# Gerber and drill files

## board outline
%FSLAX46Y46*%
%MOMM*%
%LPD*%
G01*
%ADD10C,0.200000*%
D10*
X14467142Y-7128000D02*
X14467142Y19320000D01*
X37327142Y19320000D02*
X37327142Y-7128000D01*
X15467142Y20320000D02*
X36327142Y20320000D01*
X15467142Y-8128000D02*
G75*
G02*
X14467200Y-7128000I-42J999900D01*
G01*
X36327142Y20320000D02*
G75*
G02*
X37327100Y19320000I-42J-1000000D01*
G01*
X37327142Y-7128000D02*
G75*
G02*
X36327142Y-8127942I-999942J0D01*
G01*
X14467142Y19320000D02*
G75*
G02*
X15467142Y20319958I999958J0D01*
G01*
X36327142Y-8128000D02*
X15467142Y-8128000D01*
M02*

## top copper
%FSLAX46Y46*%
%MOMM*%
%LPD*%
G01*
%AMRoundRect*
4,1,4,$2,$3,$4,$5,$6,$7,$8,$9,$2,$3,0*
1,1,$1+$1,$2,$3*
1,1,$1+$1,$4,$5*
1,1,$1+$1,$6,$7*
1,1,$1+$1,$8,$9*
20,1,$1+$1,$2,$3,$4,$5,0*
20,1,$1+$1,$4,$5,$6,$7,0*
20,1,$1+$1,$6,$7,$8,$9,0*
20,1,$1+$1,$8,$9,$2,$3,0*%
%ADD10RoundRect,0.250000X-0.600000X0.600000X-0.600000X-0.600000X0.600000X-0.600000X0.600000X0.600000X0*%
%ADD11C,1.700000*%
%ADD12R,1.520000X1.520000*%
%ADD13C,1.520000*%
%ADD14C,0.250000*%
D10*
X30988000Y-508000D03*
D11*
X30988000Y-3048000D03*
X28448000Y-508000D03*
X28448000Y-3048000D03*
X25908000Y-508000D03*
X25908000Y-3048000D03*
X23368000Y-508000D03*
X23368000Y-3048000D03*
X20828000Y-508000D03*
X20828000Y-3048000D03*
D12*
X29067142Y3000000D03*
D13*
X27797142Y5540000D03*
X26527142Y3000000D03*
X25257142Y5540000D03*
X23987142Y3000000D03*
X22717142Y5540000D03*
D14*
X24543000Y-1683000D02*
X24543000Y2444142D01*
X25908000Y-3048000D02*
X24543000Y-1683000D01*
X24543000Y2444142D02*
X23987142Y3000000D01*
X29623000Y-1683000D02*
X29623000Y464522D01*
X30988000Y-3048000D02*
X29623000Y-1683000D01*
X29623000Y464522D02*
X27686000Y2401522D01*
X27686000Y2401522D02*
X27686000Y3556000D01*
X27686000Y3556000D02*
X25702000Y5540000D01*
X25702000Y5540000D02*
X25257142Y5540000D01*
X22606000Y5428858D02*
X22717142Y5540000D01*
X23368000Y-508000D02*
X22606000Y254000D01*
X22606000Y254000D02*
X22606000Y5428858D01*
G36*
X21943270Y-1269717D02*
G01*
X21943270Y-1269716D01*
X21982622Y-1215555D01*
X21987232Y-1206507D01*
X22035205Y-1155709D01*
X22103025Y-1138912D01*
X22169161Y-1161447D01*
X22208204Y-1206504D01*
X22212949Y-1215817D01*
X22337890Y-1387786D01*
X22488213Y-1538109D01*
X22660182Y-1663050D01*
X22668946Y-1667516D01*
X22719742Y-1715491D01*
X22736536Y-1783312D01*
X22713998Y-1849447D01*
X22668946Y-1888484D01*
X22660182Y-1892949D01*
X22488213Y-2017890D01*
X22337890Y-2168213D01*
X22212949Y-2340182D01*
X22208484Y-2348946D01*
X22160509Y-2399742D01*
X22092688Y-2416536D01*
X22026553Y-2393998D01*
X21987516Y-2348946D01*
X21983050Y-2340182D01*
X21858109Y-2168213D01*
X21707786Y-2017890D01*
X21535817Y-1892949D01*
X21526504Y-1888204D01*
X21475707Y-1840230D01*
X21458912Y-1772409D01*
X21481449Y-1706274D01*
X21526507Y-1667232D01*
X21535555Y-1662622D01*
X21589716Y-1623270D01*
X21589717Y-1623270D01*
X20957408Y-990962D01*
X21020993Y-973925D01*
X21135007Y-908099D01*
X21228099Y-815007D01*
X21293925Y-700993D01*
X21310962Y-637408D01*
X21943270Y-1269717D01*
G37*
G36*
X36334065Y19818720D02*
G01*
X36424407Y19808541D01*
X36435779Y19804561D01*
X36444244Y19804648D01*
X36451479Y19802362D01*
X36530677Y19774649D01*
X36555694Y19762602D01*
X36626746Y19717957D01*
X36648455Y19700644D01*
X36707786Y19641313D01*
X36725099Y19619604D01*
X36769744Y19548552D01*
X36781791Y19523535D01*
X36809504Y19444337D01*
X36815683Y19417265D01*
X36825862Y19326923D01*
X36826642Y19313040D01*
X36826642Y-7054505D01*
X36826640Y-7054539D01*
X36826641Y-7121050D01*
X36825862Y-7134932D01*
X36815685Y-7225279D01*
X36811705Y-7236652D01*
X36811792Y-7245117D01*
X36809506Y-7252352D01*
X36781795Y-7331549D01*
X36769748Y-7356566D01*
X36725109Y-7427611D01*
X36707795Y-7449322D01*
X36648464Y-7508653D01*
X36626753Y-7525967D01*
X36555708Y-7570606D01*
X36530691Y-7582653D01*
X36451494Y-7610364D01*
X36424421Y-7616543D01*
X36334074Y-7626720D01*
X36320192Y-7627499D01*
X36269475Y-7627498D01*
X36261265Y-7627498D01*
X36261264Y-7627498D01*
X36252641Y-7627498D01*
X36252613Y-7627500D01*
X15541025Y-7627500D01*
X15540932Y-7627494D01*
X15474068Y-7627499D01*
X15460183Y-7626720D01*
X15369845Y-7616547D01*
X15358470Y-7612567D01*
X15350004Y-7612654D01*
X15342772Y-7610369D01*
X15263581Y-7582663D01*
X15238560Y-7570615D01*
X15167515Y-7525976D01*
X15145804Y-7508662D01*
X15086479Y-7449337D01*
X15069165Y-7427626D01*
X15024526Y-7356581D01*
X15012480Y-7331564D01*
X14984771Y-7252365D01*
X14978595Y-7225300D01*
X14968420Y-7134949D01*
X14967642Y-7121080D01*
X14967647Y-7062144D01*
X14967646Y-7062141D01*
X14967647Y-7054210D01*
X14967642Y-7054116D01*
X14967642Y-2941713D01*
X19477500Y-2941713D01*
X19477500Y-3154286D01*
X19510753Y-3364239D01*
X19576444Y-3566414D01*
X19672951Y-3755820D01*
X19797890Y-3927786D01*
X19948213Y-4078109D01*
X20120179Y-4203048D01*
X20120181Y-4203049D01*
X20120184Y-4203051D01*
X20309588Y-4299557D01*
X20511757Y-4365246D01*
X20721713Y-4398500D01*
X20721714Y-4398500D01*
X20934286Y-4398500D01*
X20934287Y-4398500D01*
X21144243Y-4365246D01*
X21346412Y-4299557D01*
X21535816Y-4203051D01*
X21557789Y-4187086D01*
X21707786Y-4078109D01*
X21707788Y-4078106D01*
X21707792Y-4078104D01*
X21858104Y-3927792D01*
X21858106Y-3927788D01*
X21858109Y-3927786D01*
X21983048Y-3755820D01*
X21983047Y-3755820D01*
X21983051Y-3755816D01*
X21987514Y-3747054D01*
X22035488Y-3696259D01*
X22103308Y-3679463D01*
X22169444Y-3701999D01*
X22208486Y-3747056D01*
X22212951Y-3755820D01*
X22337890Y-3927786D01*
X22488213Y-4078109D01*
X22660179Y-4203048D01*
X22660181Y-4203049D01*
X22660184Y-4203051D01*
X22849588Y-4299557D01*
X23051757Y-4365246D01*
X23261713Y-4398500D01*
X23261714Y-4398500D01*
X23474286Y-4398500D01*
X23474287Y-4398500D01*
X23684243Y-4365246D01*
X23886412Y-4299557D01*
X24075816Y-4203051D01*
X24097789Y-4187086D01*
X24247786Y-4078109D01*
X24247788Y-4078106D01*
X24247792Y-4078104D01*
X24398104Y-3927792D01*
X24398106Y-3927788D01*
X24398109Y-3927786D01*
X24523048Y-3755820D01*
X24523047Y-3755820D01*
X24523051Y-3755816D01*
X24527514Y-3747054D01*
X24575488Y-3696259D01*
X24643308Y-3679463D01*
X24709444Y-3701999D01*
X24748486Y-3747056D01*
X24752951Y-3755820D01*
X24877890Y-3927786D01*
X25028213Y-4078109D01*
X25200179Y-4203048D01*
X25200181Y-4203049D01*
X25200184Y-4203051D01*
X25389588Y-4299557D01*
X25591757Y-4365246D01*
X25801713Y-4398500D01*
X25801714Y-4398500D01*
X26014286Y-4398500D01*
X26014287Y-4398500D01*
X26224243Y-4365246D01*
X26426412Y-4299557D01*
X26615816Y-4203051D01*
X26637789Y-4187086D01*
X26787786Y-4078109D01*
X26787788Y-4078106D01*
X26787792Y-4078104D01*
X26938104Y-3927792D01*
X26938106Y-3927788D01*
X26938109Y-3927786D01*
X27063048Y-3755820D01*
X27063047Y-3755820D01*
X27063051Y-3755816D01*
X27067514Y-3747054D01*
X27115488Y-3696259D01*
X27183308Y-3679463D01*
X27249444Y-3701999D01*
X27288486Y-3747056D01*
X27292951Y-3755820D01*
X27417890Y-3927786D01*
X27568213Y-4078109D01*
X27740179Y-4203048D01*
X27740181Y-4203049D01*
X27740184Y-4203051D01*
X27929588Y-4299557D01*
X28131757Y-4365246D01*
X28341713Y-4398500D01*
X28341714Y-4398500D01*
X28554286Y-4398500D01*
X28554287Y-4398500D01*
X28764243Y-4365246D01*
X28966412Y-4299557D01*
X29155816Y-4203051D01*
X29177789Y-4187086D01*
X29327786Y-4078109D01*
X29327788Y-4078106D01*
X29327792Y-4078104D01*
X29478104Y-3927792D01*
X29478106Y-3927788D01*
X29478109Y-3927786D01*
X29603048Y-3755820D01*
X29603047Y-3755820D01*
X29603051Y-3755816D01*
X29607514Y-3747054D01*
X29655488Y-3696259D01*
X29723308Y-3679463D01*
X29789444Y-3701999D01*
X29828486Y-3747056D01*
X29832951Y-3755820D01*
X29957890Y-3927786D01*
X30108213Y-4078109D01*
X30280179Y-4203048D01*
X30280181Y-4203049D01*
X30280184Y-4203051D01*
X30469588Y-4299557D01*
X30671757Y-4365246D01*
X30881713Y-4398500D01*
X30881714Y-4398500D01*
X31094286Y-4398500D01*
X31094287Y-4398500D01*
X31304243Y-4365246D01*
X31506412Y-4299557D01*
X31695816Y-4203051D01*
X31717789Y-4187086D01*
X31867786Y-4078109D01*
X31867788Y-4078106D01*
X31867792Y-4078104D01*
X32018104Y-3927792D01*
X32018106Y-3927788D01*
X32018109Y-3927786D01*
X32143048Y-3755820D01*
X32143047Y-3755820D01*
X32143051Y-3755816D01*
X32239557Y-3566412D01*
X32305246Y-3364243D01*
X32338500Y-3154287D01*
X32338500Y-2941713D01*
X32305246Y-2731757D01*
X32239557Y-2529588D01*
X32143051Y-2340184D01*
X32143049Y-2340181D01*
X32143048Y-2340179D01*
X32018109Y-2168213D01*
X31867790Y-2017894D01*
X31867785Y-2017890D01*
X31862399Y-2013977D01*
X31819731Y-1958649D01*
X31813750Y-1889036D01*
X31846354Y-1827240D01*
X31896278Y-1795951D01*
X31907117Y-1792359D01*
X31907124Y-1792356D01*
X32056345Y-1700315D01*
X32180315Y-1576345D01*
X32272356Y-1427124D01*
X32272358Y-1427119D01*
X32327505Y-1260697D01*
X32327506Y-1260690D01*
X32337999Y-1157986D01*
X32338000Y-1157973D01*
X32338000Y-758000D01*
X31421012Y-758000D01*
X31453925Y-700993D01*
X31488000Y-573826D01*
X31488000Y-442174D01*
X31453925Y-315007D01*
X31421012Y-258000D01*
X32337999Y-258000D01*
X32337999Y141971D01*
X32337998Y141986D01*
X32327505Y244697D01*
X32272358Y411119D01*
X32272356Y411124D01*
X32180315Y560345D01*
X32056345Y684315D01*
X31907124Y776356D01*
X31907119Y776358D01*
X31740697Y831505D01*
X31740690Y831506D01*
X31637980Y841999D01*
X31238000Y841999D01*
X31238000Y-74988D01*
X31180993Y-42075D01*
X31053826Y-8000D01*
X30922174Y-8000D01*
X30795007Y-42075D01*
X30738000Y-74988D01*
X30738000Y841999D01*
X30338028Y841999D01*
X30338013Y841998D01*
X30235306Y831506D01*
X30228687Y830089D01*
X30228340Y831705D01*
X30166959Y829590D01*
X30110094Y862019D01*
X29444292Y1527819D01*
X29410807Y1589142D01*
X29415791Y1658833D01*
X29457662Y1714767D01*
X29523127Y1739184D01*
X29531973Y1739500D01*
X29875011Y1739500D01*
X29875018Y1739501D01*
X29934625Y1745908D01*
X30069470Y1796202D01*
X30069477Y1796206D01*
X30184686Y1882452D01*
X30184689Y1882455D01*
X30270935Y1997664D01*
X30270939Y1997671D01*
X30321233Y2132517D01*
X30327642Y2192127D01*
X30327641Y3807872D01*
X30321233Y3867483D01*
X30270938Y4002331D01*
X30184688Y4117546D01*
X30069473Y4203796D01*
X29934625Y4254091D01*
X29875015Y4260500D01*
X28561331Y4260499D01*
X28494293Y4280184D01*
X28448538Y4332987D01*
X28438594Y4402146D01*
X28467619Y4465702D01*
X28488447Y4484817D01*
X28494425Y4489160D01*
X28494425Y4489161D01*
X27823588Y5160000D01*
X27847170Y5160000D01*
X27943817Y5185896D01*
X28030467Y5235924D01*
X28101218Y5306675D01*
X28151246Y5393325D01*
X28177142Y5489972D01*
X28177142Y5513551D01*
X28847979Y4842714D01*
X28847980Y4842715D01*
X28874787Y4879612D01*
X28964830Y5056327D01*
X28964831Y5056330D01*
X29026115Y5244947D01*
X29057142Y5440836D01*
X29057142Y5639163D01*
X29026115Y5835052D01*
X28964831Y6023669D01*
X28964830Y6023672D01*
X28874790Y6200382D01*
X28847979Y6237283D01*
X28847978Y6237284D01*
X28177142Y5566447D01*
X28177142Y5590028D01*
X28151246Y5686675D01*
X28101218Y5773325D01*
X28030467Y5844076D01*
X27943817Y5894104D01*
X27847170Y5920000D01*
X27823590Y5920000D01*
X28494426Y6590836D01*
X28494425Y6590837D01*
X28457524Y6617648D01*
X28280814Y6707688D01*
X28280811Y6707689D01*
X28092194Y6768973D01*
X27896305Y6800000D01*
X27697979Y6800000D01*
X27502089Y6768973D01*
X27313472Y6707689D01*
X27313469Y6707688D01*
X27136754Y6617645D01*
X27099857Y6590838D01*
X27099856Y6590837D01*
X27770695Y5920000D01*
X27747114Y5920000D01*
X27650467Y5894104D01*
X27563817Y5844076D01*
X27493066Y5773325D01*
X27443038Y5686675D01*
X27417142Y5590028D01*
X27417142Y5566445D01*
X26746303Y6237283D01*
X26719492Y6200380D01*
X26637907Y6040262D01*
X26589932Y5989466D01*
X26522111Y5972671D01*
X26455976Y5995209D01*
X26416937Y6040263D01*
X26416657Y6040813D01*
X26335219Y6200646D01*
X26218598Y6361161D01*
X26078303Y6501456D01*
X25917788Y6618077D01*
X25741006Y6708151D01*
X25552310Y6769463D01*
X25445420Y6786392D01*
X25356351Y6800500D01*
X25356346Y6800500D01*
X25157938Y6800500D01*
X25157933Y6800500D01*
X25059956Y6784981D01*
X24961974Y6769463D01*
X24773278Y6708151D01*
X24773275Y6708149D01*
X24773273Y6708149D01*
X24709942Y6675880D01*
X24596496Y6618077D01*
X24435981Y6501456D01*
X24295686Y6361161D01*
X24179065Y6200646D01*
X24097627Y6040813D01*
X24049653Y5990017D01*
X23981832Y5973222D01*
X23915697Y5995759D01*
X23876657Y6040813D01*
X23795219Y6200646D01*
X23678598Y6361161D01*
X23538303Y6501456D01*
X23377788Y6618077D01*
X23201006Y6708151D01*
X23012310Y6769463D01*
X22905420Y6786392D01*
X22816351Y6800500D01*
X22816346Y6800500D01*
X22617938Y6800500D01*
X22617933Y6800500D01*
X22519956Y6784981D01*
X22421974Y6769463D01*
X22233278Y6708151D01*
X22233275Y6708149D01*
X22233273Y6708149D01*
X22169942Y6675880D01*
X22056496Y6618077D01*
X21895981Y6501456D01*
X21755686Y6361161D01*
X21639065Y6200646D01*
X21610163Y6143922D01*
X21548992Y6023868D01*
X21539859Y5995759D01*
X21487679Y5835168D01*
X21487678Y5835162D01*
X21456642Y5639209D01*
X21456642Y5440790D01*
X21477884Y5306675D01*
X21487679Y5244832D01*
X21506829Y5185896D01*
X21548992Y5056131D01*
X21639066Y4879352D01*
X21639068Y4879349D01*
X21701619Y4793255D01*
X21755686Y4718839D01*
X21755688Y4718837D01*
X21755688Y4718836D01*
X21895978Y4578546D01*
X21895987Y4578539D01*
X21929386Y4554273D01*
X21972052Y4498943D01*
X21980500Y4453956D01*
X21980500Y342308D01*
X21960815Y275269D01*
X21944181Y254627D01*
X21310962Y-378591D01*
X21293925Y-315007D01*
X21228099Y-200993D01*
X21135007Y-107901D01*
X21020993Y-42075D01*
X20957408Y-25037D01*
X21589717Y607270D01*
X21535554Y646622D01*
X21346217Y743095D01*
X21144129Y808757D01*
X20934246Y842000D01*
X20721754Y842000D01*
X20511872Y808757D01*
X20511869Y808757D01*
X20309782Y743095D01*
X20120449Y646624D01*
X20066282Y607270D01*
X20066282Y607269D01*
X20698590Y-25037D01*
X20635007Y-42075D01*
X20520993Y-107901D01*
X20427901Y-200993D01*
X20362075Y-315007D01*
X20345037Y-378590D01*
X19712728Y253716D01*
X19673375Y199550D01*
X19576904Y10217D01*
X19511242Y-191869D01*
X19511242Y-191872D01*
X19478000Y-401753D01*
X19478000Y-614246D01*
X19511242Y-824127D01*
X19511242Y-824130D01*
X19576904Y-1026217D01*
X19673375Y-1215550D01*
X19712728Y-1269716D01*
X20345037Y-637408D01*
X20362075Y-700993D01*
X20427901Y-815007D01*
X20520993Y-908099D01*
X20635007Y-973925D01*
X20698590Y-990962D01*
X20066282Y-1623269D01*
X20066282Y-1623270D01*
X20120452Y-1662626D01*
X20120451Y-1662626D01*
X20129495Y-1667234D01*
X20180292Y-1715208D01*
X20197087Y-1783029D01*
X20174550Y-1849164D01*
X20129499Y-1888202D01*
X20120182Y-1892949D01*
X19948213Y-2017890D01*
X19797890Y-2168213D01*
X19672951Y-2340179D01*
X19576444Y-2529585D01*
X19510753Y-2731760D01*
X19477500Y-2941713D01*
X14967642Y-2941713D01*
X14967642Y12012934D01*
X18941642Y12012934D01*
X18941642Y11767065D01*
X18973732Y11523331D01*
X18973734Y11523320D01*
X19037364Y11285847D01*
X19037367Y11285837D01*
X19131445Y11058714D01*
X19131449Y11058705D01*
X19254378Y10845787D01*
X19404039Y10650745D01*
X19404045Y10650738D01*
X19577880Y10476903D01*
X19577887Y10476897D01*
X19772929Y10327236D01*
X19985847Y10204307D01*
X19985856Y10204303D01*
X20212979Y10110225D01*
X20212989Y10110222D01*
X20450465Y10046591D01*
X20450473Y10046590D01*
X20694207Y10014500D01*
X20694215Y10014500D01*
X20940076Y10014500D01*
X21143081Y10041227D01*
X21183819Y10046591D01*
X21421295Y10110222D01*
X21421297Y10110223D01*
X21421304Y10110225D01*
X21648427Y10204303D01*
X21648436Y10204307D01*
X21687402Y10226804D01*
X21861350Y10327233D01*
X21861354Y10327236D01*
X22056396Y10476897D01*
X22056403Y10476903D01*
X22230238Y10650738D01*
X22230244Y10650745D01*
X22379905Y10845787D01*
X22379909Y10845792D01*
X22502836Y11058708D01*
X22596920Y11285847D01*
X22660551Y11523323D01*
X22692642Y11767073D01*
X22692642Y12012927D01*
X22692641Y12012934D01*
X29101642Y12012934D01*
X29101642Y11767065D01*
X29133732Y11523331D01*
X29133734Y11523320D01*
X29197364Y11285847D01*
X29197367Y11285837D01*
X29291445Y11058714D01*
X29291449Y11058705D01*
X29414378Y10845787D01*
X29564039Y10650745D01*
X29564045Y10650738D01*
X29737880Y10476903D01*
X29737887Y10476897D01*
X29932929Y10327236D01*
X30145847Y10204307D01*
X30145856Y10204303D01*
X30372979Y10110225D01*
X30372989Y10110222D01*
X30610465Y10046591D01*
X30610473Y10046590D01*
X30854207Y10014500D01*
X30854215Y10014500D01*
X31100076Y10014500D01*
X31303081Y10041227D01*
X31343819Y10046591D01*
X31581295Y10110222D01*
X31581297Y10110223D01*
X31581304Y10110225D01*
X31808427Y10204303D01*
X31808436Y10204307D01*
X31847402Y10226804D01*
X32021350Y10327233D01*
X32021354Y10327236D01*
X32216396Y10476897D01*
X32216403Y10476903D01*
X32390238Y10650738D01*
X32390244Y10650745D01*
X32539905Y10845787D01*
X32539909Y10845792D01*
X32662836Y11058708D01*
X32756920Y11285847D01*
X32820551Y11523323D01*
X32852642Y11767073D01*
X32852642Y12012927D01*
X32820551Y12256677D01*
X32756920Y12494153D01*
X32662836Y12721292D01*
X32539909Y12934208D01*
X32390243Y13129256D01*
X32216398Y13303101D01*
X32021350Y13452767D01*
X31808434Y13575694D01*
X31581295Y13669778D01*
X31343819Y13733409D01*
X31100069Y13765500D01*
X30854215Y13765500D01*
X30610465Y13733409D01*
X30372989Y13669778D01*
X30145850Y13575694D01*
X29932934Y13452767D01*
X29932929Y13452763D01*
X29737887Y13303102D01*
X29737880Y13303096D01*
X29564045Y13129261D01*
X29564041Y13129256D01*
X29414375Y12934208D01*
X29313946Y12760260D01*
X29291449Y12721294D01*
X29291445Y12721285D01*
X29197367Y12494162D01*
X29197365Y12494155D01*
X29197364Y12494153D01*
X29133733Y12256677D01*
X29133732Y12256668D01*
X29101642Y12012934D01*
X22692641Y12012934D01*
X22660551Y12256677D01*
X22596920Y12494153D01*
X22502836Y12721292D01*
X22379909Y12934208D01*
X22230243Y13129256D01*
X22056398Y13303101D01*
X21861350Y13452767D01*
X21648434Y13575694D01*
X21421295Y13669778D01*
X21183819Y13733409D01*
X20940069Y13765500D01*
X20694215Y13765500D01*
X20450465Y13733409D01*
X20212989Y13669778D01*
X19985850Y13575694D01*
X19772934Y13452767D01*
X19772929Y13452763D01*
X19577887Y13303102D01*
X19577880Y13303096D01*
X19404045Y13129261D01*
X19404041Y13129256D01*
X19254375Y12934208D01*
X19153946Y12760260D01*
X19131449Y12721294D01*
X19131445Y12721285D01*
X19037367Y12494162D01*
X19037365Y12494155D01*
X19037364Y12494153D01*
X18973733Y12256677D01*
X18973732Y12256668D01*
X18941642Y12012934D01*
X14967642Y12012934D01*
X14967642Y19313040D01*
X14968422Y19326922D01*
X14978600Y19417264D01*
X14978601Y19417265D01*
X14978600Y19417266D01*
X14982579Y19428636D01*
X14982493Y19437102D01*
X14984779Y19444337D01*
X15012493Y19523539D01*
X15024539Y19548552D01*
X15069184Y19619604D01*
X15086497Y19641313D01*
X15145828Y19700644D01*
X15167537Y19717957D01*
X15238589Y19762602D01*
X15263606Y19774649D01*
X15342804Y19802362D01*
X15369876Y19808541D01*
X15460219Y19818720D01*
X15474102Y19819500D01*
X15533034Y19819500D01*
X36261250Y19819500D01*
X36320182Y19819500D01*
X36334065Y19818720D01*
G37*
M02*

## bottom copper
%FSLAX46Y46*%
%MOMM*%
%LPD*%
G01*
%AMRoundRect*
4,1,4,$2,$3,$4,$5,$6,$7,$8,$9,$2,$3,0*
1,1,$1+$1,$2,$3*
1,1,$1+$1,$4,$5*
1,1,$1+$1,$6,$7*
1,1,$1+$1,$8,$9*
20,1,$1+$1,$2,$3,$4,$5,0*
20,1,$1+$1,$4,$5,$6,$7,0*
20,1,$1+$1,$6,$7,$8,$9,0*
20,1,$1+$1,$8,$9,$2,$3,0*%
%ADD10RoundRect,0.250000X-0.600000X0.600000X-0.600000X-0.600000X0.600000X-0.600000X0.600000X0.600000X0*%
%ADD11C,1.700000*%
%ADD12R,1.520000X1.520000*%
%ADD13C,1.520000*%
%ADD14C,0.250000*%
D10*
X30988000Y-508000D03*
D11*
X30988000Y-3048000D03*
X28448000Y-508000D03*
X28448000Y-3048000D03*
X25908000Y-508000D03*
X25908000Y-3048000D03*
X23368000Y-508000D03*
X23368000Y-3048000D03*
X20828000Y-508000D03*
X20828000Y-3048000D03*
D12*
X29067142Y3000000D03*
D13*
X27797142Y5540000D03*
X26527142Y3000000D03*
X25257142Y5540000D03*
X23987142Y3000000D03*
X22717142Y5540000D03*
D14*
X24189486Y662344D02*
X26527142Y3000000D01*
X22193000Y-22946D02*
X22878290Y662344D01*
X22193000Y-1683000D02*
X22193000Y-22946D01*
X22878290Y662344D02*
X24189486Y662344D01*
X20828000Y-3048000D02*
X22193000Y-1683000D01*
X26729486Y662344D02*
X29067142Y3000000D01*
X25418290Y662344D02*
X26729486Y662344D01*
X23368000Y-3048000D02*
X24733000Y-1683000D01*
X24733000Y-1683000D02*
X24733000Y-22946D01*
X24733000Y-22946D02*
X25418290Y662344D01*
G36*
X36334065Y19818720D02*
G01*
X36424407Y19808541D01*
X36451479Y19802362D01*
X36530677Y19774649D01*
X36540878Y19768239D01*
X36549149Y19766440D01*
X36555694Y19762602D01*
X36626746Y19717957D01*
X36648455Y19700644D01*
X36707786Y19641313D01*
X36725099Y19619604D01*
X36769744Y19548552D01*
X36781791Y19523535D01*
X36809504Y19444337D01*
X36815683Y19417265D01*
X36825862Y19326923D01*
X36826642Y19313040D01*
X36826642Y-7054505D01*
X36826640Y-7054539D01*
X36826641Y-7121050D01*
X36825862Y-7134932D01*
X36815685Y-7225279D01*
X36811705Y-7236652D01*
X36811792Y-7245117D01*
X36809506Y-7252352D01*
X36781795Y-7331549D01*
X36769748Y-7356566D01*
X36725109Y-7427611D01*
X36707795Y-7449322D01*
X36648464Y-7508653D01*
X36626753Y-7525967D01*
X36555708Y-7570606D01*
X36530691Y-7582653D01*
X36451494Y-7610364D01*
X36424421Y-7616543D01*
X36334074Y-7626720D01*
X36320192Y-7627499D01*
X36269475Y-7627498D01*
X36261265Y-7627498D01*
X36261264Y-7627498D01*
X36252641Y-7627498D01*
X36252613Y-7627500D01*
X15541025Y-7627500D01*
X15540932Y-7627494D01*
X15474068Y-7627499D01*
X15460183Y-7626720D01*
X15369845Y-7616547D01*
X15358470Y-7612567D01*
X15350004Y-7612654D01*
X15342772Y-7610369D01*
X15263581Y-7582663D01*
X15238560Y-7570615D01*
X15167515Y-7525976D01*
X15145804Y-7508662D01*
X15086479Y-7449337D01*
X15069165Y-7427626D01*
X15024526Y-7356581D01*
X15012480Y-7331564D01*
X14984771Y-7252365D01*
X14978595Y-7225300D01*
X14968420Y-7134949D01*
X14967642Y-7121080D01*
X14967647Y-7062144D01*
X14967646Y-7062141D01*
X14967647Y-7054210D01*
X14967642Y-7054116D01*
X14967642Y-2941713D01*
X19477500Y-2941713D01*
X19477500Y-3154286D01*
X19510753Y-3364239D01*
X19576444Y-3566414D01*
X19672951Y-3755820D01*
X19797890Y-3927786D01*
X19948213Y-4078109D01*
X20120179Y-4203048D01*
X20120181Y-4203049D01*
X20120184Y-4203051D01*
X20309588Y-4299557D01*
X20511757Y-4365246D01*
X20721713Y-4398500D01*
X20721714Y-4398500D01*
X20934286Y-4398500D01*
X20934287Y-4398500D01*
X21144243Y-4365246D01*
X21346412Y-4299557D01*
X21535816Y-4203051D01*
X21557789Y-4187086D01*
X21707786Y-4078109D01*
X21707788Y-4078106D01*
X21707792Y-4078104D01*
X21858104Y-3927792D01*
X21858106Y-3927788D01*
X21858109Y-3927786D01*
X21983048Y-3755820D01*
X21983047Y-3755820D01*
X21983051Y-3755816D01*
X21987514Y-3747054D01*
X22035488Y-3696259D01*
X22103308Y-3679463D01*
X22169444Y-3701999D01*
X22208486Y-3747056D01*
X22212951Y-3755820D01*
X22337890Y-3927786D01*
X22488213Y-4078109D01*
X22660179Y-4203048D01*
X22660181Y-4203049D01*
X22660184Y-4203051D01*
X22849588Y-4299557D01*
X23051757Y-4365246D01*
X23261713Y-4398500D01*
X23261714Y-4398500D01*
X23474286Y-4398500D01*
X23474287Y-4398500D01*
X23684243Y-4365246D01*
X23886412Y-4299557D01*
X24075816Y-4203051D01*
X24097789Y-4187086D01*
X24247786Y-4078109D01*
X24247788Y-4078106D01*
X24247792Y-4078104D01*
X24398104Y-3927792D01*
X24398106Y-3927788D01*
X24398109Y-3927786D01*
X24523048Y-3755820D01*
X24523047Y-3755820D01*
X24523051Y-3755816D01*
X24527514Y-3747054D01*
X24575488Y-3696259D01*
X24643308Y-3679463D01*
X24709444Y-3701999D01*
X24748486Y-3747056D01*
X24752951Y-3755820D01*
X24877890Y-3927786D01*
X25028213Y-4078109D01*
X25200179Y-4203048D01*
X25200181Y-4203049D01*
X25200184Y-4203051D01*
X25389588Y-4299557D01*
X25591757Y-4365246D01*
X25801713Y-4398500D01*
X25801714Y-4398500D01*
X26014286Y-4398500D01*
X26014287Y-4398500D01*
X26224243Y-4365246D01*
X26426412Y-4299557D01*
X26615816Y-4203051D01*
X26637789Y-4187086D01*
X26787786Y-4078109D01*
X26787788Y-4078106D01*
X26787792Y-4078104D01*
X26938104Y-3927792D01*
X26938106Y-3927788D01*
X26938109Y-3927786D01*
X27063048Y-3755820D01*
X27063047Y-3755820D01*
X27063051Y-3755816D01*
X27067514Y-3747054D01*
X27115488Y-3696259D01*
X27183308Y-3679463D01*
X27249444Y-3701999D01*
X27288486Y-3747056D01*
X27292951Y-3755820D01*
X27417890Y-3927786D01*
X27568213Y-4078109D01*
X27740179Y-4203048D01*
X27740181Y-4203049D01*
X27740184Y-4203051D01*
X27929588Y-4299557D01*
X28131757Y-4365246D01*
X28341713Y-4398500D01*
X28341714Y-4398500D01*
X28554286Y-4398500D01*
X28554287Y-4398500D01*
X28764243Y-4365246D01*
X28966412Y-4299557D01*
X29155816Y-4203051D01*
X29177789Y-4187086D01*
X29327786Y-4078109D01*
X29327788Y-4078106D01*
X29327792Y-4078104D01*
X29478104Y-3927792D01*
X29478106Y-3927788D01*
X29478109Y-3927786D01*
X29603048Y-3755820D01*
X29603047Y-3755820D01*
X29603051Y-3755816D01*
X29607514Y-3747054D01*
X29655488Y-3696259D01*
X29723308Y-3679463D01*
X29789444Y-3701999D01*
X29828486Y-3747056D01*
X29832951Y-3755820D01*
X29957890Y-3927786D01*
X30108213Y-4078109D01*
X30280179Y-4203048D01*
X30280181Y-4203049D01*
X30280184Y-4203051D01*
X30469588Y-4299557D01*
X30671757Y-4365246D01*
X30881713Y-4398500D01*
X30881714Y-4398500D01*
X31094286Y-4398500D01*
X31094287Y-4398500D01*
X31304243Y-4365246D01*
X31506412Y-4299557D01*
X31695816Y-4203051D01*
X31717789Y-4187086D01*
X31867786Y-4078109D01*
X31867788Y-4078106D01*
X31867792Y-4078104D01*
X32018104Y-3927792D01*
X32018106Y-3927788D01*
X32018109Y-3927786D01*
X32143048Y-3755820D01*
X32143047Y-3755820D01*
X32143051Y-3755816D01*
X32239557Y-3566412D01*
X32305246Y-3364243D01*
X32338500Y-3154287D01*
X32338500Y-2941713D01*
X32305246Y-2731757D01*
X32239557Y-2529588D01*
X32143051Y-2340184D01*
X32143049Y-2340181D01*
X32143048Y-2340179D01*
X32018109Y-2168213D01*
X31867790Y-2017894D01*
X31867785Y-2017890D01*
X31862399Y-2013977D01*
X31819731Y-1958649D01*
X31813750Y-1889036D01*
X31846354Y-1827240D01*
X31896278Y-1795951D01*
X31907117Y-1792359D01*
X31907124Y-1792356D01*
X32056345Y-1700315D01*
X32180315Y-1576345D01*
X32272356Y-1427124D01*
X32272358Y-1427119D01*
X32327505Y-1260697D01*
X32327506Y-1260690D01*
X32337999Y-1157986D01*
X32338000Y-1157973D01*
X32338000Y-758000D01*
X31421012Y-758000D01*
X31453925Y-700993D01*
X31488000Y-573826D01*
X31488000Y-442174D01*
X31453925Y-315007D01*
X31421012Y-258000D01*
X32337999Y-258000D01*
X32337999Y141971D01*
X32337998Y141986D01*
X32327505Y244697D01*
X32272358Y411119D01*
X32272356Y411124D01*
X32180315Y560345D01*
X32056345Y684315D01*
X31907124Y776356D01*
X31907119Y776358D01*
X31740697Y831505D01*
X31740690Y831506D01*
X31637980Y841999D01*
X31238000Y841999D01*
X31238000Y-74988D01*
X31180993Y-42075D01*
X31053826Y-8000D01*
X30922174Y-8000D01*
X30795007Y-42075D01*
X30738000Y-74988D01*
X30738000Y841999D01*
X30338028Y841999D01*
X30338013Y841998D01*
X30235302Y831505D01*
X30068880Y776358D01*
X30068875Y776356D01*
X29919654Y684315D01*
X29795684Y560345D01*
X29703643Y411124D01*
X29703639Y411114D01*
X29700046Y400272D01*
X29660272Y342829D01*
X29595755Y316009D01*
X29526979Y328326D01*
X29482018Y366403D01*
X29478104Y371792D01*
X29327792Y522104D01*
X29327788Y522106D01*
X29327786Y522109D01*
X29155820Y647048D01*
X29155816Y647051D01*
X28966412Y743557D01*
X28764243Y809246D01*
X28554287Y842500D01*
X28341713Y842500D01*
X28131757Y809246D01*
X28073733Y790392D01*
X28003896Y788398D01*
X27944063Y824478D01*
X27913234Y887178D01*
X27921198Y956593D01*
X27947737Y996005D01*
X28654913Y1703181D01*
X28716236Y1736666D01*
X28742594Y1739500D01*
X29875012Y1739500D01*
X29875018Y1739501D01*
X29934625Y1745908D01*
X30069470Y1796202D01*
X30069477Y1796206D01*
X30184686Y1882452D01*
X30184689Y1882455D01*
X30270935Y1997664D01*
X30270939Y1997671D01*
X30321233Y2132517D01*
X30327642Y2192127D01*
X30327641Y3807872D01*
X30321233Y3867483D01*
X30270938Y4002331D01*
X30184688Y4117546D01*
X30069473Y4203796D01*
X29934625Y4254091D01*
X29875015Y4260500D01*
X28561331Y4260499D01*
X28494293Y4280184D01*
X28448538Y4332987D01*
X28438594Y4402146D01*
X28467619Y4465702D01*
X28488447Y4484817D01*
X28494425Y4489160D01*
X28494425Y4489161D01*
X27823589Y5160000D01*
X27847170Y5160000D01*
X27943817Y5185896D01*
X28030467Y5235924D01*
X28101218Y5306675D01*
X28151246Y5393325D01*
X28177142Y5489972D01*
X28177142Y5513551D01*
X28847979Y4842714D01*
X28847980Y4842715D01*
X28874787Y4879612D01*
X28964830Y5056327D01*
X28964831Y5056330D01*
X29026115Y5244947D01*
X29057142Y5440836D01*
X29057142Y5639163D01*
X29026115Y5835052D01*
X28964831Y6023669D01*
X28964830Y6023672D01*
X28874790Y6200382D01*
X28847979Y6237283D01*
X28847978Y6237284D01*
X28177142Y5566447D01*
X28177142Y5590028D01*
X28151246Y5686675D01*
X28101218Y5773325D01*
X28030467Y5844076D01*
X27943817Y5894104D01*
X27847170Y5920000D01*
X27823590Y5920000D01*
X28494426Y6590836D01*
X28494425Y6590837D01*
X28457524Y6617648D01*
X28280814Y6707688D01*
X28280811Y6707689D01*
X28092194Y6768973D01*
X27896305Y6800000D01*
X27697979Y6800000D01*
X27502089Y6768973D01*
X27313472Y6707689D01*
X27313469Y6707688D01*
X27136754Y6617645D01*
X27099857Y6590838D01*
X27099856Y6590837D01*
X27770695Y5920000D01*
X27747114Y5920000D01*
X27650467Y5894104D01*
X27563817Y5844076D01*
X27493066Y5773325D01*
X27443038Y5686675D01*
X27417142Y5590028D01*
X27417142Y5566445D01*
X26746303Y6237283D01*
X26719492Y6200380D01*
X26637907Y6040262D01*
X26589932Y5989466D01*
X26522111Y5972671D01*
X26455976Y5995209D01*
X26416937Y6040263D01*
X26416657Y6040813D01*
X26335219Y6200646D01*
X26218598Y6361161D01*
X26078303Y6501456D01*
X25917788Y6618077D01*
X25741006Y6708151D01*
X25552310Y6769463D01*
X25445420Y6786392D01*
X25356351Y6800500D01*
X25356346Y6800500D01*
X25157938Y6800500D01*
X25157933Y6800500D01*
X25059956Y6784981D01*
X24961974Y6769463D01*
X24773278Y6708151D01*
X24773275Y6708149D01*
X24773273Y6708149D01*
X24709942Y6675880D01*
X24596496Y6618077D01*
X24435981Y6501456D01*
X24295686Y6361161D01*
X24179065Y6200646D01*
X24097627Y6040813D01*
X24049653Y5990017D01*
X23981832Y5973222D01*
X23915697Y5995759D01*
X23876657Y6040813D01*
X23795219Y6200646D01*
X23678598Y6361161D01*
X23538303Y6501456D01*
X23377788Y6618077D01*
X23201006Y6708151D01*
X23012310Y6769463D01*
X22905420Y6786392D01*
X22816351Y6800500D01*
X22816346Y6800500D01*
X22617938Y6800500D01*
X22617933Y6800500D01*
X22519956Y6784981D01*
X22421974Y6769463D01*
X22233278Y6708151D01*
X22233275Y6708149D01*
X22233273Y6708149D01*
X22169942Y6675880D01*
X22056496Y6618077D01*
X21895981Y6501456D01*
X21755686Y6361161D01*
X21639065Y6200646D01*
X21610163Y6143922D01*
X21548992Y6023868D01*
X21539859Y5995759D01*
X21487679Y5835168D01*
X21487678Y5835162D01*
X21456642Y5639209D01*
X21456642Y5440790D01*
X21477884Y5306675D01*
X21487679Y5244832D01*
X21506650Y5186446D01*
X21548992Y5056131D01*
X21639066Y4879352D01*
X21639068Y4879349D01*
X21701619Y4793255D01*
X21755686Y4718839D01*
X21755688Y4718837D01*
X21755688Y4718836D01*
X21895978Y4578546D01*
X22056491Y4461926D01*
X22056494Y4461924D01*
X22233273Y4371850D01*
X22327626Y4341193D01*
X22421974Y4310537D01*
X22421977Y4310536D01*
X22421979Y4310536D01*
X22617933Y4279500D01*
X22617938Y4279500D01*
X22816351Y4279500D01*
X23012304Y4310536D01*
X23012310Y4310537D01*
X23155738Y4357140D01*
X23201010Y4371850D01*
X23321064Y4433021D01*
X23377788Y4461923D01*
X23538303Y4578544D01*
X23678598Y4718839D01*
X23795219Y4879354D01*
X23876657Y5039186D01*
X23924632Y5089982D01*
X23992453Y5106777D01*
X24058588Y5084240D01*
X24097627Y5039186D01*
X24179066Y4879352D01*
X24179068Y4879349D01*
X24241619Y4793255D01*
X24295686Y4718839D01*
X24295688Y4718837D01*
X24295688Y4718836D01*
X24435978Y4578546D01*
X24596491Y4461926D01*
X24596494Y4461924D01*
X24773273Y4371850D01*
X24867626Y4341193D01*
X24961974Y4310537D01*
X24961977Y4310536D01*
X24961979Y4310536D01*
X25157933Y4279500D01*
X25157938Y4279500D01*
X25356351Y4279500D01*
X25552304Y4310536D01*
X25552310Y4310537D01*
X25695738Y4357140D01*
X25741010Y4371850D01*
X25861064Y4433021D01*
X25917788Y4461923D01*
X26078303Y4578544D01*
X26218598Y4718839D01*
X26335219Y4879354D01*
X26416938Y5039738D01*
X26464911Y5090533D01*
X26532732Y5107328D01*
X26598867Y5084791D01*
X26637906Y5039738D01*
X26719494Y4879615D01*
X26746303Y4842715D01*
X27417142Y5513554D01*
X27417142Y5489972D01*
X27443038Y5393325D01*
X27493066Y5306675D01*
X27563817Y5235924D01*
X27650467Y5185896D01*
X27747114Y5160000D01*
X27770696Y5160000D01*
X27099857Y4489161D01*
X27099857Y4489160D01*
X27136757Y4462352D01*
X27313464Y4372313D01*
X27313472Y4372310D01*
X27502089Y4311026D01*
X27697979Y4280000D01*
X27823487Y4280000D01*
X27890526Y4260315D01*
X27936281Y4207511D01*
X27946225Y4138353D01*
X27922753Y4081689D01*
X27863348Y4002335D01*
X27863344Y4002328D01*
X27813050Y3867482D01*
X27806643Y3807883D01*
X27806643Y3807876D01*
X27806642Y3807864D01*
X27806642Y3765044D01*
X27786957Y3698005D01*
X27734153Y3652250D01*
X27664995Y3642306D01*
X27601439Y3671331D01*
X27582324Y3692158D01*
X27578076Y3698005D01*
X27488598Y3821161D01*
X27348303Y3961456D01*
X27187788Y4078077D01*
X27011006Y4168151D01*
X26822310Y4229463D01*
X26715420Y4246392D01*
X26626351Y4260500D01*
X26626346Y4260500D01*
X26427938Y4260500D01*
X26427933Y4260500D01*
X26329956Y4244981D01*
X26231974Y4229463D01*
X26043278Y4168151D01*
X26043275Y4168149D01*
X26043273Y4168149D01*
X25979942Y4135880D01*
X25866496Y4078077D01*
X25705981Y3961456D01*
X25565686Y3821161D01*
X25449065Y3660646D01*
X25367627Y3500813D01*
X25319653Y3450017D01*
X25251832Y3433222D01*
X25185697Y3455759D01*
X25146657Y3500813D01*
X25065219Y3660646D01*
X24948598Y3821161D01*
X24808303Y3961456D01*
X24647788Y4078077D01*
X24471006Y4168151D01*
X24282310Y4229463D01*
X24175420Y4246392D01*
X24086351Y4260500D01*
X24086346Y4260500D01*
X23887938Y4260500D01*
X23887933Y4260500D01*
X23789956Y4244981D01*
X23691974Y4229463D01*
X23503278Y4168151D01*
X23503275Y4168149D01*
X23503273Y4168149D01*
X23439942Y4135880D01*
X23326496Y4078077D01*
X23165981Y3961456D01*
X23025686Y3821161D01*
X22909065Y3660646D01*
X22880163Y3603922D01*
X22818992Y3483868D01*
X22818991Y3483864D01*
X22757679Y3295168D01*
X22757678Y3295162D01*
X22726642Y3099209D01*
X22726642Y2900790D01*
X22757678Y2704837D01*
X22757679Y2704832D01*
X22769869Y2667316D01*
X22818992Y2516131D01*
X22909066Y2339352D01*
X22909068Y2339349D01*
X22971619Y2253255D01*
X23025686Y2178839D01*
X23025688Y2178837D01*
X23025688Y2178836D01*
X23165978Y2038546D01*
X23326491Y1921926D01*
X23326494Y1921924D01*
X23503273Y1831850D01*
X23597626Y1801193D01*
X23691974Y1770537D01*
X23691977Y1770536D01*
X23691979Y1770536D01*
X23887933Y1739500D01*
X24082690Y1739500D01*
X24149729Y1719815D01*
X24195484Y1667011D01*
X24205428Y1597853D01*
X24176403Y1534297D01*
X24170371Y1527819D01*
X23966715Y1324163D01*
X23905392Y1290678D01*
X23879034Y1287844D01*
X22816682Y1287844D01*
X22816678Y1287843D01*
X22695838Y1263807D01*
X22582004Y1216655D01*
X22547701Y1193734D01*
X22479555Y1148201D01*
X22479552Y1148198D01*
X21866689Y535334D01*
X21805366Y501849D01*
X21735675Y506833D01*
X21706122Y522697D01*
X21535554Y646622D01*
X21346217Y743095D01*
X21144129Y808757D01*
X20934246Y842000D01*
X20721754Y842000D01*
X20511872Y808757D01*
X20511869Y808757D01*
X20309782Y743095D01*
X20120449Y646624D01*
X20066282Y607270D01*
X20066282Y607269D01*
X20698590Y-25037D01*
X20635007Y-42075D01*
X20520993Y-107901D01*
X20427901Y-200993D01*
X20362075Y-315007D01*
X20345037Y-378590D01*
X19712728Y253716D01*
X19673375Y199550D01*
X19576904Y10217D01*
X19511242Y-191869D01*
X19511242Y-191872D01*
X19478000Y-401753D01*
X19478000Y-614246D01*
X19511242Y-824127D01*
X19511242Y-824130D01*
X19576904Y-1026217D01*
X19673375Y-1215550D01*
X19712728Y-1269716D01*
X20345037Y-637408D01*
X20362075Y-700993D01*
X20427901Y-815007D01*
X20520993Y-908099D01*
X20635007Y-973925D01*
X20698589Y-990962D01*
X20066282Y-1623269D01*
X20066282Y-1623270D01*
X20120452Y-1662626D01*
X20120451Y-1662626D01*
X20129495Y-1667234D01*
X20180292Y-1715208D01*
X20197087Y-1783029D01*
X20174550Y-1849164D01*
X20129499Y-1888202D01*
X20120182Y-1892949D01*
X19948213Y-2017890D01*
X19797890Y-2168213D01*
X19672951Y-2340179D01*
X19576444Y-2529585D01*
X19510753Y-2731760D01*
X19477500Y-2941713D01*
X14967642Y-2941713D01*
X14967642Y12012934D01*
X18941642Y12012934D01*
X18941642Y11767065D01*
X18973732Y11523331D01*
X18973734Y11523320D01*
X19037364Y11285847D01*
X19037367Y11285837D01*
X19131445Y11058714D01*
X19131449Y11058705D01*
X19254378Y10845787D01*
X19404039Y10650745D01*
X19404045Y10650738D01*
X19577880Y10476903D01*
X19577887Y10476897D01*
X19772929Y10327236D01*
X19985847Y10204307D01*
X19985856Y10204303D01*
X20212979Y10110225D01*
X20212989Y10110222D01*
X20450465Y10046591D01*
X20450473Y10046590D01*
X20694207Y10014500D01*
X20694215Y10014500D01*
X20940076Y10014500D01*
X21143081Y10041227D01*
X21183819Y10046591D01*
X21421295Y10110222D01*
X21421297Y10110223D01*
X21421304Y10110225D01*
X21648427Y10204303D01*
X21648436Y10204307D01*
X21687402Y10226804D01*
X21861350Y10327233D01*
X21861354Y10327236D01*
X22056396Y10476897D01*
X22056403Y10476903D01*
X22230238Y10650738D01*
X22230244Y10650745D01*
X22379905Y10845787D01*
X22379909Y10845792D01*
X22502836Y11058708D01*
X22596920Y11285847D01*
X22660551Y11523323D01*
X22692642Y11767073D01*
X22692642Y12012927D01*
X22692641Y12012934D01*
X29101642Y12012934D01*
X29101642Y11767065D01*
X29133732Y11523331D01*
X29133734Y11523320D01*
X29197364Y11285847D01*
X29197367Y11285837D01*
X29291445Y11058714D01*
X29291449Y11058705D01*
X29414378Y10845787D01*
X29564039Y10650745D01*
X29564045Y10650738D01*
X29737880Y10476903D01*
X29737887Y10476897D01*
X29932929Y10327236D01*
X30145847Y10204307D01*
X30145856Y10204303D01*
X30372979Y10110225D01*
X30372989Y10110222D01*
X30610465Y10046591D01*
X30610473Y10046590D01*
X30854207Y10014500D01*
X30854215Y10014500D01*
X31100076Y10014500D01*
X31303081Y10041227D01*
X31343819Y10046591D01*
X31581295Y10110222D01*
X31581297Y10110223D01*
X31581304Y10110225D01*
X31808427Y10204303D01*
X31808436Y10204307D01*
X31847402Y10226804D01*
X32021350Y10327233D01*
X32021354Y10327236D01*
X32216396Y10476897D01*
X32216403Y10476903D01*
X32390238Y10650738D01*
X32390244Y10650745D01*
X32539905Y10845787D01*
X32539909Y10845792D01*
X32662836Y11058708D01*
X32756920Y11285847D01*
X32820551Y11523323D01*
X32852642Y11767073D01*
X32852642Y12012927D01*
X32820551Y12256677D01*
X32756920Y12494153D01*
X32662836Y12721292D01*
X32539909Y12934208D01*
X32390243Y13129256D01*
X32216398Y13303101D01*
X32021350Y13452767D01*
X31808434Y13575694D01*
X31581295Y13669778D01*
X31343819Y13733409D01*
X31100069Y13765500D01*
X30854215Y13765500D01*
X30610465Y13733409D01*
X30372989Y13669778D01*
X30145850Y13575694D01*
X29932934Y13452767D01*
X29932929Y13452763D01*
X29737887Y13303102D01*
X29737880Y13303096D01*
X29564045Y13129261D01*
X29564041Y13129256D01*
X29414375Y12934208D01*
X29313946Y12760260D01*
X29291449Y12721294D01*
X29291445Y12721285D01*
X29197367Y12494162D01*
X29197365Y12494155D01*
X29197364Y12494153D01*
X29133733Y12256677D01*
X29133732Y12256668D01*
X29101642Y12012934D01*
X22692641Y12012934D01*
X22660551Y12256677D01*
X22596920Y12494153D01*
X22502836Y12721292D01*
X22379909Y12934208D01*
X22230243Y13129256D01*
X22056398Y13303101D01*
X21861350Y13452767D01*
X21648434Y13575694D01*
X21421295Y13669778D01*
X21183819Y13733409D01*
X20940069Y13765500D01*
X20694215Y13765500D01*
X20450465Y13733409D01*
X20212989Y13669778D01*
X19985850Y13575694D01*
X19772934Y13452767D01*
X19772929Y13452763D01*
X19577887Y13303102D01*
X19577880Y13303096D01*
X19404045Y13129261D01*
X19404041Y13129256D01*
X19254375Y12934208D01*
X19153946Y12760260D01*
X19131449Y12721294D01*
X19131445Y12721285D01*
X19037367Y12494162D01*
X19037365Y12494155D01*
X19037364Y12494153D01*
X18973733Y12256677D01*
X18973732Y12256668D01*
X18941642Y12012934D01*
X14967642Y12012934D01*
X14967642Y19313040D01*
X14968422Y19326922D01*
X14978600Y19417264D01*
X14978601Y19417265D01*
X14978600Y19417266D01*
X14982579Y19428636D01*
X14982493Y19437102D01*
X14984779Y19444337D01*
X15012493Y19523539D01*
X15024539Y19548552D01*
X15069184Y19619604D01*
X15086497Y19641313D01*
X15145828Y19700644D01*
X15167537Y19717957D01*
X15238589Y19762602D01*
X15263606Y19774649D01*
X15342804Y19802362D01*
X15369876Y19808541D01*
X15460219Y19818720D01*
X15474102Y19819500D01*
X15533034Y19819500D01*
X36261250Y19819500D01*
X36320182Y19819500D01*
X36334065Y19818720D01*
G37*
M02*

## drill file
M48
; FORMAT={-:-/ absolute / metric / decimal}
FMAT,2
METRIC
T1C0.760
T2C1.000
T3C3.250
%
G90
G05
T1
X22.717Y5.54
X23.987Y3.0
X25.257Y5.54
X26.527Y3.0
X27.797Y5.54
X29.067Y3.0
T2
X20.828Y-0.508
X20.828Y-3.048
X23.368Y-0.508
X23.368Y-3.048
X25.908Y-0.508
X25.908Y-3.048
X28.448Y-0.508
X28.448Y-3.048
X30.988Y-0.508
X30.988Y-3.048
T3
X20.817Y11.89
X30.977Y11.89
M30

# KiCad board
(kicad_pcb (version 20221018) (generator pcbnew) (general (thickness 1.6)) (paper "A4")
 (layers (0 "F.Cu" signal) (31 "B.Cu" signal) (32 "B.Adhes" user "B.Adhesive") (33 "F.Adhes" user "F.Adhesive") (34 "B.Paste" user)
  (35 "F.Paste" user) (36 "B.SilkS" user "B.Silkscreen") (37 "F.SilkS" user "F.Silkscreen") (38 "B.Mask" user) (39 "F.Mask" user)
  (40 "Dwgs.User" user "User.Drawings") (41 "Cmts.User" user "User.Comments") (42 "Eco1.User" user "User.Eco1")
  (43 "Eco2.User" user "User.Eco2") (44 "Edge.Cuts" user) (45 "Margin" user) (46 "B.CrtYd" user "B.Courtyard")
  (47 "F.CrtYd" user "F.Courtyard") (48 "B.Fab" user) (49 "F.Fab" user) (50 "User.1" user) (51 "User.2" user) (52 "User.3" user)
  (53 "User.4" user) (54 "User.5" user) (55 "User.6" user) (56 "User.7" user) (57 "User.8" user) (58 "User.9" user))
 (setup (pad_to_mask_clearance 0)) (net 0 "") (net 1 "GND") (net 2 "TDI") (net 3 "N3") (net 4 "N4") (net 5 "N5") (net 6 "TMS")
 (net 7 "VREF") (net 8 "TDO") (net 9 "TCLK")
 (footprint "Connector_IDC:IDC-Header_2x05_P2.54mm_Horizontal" (layer "F.Cu") (at 25.908 6.723 -90)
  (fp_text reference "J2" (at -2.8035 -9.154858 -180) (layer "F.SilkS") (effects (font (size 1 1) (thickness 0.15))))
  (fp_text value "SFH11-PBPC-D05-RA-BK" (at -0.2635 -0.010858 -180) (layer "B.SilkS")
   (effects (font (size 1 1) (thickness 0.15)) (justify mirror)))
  (pad "1" thru_hole roundrect (at -6.215 -5.08 270) (size 1.7 1.7) (drill 1) (layers "*.Cu" "*.Mask") (roundrect_rratio 0.147059)
   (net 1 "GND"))
  (pad "2" thru_hole circle (at -3.675 -5.08 270) (size 1.7 1.7) (drill 1) (layers "*.Cu" "*.Mask") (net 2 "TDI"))
  (pad "3" thru_hole circle (at -6.215 -2.54 270) (size 1.7 1.7) (drill 1) (layers "*.Cu" "*.Mask") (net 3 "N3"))
  (pad "4" thru_hole circle (at -3.675 -2.54 270) (size 1.7 1.7) (drill 1) (layers "*.Cu" "*.Mask") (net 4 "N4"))
  (pad "5" thru_hole circle (at -6.215 0 270) (size 1.7 1.7) (drill 1) (layers "*.Cu" "*.Mask") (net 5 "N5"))
  (pad "6" thru_hole circle (at -3.675 0 270) (size 1.7 1.7) (drill 1) (layers "*.Cu" "*.Mask") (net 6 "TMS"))
  (pad "7" thru_hole circle (at -6.215 2.54 270) (size 1.7 1.7) (drill 1) (layers "*.Cu" "*.Mask") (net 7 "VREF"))
  (pad "8" thru_hole circle (at -3.675 2.54 270) (size 1.7 1.7) (drill 1) (layers "*.Cu" "*.Mask") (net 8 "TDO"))
  (pad "9" thru_hole circle (at -6.215 5.08 270) (size 1.7 1.7) (drill 1) (layers "*.Cu" "*.Mask") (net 1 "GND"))
  (pad "10" thru_hole circle (at -3.675 5.08 270) (size 1.7 1.7) (drill 1) (layers "*.Cu" "*.Mask") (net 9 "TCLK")))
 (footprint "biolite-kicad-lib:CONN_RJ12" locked (layer "F.Cu") (at 29.067142 -3 180)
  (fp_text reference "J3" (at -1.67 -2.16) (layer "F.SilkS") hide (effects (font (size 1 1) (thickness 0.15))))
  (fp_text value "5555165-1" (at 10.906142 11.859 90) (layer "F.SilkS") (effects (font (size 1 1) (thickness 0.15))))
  (pad "" np_thru_hole circle locked (at -1.91 8.89 180) (size 3.25 3.25) (drill 3.25) (layers "*.Cu" "*.Mask"))
  (pad "" np_thru_hole circle locked (at 8.25 8.89 180) (size 3.25 3.25) (drill 3.25) (layers "*.Cu" "*.Mask"))
  (pad "1" thru_hole rect locked (at 0 0 180) (size 1.52 1.52) (drill 0.76) (layers "*.Cu" "*.Mask") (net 8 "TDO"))
  (pad "2" thru_hole circle locked (at 1.27 2.54 180) (size 1.52 1.52) (drill 0.76) (layers "*.Cu" "*.Mask") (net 1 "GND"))
  (pad "3" thru_hole circle locked (at 2.54 0 180) (size 1.52 1.52) (drill 0.76) (layers "*.Cu" "*.Mask") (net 9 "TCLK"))
  (pad "4" thru_hole circle locked (at 3.81 2.54 180) (size 1.52 1.52) (drill 0.76) (layers "*.Cu" "*.Mask") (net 2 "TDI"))
  (pad "5" thru_hole circle locked (at 5.08 0 180) (size 1.52 1.52) (drill 0.76) (layers "*.Cu" "*.Mask") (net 6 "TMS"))
  (pad "6" thru_hole circle locked (at 6.35 2.54 180) (size 1.52 1.52) (drill 0.76) (layers "*.Cu" "*.Mask") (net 7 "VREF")))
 (gr_line (start 14.467142 7.128) (end 14.467142 -19.32) (stroke (width 0.2) (type default)) (layer "Edge.Cuts"))
 (gr_line (start 37.327142 -19.32) (end 37.327142 7.128) (stroke (width 0.2) (type default)) (layer "Edge.Cuts"))
 (gr_line (start 15.467142 -20.32) (end 36.327142 -20.32) (stroke (width 0.2) (type default)) (layer "Edge.Cuts"))
 (gr_arc (start 15.467142 8.128) (mid 14.760008 7.835122) (end 14.467142 7.128) (stroke (width 0.2) (type default)) (layer "Edge.Cuts"))
 (gr_arc (start 36.327142 -20.32) (mid 37.034249 -20.027107) (end 37.327142 -19.32) (stroke (width 0.2) (type default)) (layer "Edge.Cuts"))
 (gr_arc (start 37.327142 7.128) (mid 37.034251 7.835122) (end 36.327142 8.128) (stroke (width 0.2) (type default)) (layer "Edge.Cuts"))
 (gr_arc (start 14.467142 -19.32) (mid 14.760035 -20.027107) (end 15.467142 -20.32) (stroke (width 0.2) (type default)) (layer "Edge.Cuts"))
 (gr_line (start 36.327142 8.128) (end 15.467142 8.128) (stroke (width 0.2) (type default)) (layer "Edge.Cuts"))
 (segment (start 24.189486 -0.662344) (end 26.527142 -3) (width 0.25) (layer "B.Cu") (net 9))
 (segment (start 22.193 0.022946) (end 22.87829 -0.662344) (width 0.25) (layer "B.Cu") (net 9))
 (segment (start 22.193 1.683) (end 22.193 0.022946) (width 0.25) (layer "B.Cu") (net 9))
 (segment (start 22.87829 -0.662344) (end 24.189486 -0.662344) (width 0.25) (layer "B.Cu") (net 9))
 (segment (start 20.828 3.048) (end 22.193 1.683) (width 0.25) (layer "B.Cu") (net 9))
 (segment (start 26.729486 -0.662344) (end 29.067142 -3) (width 0.25) (layer "B.Cu") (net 8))
 (segment (start 25.41829 -0.662344) (end 26.729486 -0.662344) (width 0.25) (layer "B.Cu") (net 8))
 (segment (start 23.368 3.048) (end 24.733 1.683) (width 0.25) (layer "B.Cu") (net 8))
 (segment (start 24.733 1.683) (end 24.733 0.022946) (width 0.25) (layer "B.Cu") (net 8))
 (segment (start 24.733 0.022946) (end 25.41829 -0.662344) (width 0.25) (layer "B.Cu") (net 8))
 (segment (start 24.543 1.683) (end 24.543 -2.444142) (width 0.25) (layer "F.Cu") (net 6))
 (segment (start 25.908 3.048) (end 24.543 1.683) (width 0.25) (layer "F.Cu") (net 6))
 (segment (start 24.543 -2.444142) (end 23.987142 -3) (width 0.25) (layer "F.Cu") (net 6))
 (segment (start 29.623 1.683) (end 29.623 -0.464522) (width 0.25) (layer "F.Cu") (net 2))
 (segment (start 30.988 3.048) (end 29.623 1.683) (width 0.25) (layer "F.Cu") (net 2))
 (segment (start 29.623 -0.464522) (end 27.686 -2.401522) (width 0.25) (layer "F.Cu") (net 2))
 (segment (start 27.686 -2.401522) (end 27.686 -3.556) (width 0.25) (layer "F.Cu") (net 2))
 (segment (start 27.686 -3.556) (end 25.702 -5.54) (width 0.25) (layer "F.Cu") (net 2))
 (segment (start 25.702 -5.54) (end 25.257142 -5.54) (width 0.25) (layer "F.Cu") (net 2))
 (segment (start 22.606 -5.428858) (end 22.717142 -5.54) (width 0.25) (layer "F.Cu") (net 7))
 (segment (start 23.368 0.508) (end 22.606 -0.254) (width 0.25) (layer "F.Cu") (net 7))
 (segment (start 22.606 -0.254) (end 22.606 -5.428858) (width 0.25) (layer "F.Cu") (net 7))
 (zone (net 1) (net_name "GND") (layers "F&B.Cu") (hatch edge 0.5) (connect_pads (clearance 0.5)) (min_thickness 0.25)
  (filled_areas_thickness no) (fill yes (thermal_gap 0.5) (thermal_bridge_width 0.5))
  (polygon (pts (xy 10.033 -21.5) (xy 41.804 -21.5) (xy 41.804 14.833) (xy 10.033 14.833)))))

